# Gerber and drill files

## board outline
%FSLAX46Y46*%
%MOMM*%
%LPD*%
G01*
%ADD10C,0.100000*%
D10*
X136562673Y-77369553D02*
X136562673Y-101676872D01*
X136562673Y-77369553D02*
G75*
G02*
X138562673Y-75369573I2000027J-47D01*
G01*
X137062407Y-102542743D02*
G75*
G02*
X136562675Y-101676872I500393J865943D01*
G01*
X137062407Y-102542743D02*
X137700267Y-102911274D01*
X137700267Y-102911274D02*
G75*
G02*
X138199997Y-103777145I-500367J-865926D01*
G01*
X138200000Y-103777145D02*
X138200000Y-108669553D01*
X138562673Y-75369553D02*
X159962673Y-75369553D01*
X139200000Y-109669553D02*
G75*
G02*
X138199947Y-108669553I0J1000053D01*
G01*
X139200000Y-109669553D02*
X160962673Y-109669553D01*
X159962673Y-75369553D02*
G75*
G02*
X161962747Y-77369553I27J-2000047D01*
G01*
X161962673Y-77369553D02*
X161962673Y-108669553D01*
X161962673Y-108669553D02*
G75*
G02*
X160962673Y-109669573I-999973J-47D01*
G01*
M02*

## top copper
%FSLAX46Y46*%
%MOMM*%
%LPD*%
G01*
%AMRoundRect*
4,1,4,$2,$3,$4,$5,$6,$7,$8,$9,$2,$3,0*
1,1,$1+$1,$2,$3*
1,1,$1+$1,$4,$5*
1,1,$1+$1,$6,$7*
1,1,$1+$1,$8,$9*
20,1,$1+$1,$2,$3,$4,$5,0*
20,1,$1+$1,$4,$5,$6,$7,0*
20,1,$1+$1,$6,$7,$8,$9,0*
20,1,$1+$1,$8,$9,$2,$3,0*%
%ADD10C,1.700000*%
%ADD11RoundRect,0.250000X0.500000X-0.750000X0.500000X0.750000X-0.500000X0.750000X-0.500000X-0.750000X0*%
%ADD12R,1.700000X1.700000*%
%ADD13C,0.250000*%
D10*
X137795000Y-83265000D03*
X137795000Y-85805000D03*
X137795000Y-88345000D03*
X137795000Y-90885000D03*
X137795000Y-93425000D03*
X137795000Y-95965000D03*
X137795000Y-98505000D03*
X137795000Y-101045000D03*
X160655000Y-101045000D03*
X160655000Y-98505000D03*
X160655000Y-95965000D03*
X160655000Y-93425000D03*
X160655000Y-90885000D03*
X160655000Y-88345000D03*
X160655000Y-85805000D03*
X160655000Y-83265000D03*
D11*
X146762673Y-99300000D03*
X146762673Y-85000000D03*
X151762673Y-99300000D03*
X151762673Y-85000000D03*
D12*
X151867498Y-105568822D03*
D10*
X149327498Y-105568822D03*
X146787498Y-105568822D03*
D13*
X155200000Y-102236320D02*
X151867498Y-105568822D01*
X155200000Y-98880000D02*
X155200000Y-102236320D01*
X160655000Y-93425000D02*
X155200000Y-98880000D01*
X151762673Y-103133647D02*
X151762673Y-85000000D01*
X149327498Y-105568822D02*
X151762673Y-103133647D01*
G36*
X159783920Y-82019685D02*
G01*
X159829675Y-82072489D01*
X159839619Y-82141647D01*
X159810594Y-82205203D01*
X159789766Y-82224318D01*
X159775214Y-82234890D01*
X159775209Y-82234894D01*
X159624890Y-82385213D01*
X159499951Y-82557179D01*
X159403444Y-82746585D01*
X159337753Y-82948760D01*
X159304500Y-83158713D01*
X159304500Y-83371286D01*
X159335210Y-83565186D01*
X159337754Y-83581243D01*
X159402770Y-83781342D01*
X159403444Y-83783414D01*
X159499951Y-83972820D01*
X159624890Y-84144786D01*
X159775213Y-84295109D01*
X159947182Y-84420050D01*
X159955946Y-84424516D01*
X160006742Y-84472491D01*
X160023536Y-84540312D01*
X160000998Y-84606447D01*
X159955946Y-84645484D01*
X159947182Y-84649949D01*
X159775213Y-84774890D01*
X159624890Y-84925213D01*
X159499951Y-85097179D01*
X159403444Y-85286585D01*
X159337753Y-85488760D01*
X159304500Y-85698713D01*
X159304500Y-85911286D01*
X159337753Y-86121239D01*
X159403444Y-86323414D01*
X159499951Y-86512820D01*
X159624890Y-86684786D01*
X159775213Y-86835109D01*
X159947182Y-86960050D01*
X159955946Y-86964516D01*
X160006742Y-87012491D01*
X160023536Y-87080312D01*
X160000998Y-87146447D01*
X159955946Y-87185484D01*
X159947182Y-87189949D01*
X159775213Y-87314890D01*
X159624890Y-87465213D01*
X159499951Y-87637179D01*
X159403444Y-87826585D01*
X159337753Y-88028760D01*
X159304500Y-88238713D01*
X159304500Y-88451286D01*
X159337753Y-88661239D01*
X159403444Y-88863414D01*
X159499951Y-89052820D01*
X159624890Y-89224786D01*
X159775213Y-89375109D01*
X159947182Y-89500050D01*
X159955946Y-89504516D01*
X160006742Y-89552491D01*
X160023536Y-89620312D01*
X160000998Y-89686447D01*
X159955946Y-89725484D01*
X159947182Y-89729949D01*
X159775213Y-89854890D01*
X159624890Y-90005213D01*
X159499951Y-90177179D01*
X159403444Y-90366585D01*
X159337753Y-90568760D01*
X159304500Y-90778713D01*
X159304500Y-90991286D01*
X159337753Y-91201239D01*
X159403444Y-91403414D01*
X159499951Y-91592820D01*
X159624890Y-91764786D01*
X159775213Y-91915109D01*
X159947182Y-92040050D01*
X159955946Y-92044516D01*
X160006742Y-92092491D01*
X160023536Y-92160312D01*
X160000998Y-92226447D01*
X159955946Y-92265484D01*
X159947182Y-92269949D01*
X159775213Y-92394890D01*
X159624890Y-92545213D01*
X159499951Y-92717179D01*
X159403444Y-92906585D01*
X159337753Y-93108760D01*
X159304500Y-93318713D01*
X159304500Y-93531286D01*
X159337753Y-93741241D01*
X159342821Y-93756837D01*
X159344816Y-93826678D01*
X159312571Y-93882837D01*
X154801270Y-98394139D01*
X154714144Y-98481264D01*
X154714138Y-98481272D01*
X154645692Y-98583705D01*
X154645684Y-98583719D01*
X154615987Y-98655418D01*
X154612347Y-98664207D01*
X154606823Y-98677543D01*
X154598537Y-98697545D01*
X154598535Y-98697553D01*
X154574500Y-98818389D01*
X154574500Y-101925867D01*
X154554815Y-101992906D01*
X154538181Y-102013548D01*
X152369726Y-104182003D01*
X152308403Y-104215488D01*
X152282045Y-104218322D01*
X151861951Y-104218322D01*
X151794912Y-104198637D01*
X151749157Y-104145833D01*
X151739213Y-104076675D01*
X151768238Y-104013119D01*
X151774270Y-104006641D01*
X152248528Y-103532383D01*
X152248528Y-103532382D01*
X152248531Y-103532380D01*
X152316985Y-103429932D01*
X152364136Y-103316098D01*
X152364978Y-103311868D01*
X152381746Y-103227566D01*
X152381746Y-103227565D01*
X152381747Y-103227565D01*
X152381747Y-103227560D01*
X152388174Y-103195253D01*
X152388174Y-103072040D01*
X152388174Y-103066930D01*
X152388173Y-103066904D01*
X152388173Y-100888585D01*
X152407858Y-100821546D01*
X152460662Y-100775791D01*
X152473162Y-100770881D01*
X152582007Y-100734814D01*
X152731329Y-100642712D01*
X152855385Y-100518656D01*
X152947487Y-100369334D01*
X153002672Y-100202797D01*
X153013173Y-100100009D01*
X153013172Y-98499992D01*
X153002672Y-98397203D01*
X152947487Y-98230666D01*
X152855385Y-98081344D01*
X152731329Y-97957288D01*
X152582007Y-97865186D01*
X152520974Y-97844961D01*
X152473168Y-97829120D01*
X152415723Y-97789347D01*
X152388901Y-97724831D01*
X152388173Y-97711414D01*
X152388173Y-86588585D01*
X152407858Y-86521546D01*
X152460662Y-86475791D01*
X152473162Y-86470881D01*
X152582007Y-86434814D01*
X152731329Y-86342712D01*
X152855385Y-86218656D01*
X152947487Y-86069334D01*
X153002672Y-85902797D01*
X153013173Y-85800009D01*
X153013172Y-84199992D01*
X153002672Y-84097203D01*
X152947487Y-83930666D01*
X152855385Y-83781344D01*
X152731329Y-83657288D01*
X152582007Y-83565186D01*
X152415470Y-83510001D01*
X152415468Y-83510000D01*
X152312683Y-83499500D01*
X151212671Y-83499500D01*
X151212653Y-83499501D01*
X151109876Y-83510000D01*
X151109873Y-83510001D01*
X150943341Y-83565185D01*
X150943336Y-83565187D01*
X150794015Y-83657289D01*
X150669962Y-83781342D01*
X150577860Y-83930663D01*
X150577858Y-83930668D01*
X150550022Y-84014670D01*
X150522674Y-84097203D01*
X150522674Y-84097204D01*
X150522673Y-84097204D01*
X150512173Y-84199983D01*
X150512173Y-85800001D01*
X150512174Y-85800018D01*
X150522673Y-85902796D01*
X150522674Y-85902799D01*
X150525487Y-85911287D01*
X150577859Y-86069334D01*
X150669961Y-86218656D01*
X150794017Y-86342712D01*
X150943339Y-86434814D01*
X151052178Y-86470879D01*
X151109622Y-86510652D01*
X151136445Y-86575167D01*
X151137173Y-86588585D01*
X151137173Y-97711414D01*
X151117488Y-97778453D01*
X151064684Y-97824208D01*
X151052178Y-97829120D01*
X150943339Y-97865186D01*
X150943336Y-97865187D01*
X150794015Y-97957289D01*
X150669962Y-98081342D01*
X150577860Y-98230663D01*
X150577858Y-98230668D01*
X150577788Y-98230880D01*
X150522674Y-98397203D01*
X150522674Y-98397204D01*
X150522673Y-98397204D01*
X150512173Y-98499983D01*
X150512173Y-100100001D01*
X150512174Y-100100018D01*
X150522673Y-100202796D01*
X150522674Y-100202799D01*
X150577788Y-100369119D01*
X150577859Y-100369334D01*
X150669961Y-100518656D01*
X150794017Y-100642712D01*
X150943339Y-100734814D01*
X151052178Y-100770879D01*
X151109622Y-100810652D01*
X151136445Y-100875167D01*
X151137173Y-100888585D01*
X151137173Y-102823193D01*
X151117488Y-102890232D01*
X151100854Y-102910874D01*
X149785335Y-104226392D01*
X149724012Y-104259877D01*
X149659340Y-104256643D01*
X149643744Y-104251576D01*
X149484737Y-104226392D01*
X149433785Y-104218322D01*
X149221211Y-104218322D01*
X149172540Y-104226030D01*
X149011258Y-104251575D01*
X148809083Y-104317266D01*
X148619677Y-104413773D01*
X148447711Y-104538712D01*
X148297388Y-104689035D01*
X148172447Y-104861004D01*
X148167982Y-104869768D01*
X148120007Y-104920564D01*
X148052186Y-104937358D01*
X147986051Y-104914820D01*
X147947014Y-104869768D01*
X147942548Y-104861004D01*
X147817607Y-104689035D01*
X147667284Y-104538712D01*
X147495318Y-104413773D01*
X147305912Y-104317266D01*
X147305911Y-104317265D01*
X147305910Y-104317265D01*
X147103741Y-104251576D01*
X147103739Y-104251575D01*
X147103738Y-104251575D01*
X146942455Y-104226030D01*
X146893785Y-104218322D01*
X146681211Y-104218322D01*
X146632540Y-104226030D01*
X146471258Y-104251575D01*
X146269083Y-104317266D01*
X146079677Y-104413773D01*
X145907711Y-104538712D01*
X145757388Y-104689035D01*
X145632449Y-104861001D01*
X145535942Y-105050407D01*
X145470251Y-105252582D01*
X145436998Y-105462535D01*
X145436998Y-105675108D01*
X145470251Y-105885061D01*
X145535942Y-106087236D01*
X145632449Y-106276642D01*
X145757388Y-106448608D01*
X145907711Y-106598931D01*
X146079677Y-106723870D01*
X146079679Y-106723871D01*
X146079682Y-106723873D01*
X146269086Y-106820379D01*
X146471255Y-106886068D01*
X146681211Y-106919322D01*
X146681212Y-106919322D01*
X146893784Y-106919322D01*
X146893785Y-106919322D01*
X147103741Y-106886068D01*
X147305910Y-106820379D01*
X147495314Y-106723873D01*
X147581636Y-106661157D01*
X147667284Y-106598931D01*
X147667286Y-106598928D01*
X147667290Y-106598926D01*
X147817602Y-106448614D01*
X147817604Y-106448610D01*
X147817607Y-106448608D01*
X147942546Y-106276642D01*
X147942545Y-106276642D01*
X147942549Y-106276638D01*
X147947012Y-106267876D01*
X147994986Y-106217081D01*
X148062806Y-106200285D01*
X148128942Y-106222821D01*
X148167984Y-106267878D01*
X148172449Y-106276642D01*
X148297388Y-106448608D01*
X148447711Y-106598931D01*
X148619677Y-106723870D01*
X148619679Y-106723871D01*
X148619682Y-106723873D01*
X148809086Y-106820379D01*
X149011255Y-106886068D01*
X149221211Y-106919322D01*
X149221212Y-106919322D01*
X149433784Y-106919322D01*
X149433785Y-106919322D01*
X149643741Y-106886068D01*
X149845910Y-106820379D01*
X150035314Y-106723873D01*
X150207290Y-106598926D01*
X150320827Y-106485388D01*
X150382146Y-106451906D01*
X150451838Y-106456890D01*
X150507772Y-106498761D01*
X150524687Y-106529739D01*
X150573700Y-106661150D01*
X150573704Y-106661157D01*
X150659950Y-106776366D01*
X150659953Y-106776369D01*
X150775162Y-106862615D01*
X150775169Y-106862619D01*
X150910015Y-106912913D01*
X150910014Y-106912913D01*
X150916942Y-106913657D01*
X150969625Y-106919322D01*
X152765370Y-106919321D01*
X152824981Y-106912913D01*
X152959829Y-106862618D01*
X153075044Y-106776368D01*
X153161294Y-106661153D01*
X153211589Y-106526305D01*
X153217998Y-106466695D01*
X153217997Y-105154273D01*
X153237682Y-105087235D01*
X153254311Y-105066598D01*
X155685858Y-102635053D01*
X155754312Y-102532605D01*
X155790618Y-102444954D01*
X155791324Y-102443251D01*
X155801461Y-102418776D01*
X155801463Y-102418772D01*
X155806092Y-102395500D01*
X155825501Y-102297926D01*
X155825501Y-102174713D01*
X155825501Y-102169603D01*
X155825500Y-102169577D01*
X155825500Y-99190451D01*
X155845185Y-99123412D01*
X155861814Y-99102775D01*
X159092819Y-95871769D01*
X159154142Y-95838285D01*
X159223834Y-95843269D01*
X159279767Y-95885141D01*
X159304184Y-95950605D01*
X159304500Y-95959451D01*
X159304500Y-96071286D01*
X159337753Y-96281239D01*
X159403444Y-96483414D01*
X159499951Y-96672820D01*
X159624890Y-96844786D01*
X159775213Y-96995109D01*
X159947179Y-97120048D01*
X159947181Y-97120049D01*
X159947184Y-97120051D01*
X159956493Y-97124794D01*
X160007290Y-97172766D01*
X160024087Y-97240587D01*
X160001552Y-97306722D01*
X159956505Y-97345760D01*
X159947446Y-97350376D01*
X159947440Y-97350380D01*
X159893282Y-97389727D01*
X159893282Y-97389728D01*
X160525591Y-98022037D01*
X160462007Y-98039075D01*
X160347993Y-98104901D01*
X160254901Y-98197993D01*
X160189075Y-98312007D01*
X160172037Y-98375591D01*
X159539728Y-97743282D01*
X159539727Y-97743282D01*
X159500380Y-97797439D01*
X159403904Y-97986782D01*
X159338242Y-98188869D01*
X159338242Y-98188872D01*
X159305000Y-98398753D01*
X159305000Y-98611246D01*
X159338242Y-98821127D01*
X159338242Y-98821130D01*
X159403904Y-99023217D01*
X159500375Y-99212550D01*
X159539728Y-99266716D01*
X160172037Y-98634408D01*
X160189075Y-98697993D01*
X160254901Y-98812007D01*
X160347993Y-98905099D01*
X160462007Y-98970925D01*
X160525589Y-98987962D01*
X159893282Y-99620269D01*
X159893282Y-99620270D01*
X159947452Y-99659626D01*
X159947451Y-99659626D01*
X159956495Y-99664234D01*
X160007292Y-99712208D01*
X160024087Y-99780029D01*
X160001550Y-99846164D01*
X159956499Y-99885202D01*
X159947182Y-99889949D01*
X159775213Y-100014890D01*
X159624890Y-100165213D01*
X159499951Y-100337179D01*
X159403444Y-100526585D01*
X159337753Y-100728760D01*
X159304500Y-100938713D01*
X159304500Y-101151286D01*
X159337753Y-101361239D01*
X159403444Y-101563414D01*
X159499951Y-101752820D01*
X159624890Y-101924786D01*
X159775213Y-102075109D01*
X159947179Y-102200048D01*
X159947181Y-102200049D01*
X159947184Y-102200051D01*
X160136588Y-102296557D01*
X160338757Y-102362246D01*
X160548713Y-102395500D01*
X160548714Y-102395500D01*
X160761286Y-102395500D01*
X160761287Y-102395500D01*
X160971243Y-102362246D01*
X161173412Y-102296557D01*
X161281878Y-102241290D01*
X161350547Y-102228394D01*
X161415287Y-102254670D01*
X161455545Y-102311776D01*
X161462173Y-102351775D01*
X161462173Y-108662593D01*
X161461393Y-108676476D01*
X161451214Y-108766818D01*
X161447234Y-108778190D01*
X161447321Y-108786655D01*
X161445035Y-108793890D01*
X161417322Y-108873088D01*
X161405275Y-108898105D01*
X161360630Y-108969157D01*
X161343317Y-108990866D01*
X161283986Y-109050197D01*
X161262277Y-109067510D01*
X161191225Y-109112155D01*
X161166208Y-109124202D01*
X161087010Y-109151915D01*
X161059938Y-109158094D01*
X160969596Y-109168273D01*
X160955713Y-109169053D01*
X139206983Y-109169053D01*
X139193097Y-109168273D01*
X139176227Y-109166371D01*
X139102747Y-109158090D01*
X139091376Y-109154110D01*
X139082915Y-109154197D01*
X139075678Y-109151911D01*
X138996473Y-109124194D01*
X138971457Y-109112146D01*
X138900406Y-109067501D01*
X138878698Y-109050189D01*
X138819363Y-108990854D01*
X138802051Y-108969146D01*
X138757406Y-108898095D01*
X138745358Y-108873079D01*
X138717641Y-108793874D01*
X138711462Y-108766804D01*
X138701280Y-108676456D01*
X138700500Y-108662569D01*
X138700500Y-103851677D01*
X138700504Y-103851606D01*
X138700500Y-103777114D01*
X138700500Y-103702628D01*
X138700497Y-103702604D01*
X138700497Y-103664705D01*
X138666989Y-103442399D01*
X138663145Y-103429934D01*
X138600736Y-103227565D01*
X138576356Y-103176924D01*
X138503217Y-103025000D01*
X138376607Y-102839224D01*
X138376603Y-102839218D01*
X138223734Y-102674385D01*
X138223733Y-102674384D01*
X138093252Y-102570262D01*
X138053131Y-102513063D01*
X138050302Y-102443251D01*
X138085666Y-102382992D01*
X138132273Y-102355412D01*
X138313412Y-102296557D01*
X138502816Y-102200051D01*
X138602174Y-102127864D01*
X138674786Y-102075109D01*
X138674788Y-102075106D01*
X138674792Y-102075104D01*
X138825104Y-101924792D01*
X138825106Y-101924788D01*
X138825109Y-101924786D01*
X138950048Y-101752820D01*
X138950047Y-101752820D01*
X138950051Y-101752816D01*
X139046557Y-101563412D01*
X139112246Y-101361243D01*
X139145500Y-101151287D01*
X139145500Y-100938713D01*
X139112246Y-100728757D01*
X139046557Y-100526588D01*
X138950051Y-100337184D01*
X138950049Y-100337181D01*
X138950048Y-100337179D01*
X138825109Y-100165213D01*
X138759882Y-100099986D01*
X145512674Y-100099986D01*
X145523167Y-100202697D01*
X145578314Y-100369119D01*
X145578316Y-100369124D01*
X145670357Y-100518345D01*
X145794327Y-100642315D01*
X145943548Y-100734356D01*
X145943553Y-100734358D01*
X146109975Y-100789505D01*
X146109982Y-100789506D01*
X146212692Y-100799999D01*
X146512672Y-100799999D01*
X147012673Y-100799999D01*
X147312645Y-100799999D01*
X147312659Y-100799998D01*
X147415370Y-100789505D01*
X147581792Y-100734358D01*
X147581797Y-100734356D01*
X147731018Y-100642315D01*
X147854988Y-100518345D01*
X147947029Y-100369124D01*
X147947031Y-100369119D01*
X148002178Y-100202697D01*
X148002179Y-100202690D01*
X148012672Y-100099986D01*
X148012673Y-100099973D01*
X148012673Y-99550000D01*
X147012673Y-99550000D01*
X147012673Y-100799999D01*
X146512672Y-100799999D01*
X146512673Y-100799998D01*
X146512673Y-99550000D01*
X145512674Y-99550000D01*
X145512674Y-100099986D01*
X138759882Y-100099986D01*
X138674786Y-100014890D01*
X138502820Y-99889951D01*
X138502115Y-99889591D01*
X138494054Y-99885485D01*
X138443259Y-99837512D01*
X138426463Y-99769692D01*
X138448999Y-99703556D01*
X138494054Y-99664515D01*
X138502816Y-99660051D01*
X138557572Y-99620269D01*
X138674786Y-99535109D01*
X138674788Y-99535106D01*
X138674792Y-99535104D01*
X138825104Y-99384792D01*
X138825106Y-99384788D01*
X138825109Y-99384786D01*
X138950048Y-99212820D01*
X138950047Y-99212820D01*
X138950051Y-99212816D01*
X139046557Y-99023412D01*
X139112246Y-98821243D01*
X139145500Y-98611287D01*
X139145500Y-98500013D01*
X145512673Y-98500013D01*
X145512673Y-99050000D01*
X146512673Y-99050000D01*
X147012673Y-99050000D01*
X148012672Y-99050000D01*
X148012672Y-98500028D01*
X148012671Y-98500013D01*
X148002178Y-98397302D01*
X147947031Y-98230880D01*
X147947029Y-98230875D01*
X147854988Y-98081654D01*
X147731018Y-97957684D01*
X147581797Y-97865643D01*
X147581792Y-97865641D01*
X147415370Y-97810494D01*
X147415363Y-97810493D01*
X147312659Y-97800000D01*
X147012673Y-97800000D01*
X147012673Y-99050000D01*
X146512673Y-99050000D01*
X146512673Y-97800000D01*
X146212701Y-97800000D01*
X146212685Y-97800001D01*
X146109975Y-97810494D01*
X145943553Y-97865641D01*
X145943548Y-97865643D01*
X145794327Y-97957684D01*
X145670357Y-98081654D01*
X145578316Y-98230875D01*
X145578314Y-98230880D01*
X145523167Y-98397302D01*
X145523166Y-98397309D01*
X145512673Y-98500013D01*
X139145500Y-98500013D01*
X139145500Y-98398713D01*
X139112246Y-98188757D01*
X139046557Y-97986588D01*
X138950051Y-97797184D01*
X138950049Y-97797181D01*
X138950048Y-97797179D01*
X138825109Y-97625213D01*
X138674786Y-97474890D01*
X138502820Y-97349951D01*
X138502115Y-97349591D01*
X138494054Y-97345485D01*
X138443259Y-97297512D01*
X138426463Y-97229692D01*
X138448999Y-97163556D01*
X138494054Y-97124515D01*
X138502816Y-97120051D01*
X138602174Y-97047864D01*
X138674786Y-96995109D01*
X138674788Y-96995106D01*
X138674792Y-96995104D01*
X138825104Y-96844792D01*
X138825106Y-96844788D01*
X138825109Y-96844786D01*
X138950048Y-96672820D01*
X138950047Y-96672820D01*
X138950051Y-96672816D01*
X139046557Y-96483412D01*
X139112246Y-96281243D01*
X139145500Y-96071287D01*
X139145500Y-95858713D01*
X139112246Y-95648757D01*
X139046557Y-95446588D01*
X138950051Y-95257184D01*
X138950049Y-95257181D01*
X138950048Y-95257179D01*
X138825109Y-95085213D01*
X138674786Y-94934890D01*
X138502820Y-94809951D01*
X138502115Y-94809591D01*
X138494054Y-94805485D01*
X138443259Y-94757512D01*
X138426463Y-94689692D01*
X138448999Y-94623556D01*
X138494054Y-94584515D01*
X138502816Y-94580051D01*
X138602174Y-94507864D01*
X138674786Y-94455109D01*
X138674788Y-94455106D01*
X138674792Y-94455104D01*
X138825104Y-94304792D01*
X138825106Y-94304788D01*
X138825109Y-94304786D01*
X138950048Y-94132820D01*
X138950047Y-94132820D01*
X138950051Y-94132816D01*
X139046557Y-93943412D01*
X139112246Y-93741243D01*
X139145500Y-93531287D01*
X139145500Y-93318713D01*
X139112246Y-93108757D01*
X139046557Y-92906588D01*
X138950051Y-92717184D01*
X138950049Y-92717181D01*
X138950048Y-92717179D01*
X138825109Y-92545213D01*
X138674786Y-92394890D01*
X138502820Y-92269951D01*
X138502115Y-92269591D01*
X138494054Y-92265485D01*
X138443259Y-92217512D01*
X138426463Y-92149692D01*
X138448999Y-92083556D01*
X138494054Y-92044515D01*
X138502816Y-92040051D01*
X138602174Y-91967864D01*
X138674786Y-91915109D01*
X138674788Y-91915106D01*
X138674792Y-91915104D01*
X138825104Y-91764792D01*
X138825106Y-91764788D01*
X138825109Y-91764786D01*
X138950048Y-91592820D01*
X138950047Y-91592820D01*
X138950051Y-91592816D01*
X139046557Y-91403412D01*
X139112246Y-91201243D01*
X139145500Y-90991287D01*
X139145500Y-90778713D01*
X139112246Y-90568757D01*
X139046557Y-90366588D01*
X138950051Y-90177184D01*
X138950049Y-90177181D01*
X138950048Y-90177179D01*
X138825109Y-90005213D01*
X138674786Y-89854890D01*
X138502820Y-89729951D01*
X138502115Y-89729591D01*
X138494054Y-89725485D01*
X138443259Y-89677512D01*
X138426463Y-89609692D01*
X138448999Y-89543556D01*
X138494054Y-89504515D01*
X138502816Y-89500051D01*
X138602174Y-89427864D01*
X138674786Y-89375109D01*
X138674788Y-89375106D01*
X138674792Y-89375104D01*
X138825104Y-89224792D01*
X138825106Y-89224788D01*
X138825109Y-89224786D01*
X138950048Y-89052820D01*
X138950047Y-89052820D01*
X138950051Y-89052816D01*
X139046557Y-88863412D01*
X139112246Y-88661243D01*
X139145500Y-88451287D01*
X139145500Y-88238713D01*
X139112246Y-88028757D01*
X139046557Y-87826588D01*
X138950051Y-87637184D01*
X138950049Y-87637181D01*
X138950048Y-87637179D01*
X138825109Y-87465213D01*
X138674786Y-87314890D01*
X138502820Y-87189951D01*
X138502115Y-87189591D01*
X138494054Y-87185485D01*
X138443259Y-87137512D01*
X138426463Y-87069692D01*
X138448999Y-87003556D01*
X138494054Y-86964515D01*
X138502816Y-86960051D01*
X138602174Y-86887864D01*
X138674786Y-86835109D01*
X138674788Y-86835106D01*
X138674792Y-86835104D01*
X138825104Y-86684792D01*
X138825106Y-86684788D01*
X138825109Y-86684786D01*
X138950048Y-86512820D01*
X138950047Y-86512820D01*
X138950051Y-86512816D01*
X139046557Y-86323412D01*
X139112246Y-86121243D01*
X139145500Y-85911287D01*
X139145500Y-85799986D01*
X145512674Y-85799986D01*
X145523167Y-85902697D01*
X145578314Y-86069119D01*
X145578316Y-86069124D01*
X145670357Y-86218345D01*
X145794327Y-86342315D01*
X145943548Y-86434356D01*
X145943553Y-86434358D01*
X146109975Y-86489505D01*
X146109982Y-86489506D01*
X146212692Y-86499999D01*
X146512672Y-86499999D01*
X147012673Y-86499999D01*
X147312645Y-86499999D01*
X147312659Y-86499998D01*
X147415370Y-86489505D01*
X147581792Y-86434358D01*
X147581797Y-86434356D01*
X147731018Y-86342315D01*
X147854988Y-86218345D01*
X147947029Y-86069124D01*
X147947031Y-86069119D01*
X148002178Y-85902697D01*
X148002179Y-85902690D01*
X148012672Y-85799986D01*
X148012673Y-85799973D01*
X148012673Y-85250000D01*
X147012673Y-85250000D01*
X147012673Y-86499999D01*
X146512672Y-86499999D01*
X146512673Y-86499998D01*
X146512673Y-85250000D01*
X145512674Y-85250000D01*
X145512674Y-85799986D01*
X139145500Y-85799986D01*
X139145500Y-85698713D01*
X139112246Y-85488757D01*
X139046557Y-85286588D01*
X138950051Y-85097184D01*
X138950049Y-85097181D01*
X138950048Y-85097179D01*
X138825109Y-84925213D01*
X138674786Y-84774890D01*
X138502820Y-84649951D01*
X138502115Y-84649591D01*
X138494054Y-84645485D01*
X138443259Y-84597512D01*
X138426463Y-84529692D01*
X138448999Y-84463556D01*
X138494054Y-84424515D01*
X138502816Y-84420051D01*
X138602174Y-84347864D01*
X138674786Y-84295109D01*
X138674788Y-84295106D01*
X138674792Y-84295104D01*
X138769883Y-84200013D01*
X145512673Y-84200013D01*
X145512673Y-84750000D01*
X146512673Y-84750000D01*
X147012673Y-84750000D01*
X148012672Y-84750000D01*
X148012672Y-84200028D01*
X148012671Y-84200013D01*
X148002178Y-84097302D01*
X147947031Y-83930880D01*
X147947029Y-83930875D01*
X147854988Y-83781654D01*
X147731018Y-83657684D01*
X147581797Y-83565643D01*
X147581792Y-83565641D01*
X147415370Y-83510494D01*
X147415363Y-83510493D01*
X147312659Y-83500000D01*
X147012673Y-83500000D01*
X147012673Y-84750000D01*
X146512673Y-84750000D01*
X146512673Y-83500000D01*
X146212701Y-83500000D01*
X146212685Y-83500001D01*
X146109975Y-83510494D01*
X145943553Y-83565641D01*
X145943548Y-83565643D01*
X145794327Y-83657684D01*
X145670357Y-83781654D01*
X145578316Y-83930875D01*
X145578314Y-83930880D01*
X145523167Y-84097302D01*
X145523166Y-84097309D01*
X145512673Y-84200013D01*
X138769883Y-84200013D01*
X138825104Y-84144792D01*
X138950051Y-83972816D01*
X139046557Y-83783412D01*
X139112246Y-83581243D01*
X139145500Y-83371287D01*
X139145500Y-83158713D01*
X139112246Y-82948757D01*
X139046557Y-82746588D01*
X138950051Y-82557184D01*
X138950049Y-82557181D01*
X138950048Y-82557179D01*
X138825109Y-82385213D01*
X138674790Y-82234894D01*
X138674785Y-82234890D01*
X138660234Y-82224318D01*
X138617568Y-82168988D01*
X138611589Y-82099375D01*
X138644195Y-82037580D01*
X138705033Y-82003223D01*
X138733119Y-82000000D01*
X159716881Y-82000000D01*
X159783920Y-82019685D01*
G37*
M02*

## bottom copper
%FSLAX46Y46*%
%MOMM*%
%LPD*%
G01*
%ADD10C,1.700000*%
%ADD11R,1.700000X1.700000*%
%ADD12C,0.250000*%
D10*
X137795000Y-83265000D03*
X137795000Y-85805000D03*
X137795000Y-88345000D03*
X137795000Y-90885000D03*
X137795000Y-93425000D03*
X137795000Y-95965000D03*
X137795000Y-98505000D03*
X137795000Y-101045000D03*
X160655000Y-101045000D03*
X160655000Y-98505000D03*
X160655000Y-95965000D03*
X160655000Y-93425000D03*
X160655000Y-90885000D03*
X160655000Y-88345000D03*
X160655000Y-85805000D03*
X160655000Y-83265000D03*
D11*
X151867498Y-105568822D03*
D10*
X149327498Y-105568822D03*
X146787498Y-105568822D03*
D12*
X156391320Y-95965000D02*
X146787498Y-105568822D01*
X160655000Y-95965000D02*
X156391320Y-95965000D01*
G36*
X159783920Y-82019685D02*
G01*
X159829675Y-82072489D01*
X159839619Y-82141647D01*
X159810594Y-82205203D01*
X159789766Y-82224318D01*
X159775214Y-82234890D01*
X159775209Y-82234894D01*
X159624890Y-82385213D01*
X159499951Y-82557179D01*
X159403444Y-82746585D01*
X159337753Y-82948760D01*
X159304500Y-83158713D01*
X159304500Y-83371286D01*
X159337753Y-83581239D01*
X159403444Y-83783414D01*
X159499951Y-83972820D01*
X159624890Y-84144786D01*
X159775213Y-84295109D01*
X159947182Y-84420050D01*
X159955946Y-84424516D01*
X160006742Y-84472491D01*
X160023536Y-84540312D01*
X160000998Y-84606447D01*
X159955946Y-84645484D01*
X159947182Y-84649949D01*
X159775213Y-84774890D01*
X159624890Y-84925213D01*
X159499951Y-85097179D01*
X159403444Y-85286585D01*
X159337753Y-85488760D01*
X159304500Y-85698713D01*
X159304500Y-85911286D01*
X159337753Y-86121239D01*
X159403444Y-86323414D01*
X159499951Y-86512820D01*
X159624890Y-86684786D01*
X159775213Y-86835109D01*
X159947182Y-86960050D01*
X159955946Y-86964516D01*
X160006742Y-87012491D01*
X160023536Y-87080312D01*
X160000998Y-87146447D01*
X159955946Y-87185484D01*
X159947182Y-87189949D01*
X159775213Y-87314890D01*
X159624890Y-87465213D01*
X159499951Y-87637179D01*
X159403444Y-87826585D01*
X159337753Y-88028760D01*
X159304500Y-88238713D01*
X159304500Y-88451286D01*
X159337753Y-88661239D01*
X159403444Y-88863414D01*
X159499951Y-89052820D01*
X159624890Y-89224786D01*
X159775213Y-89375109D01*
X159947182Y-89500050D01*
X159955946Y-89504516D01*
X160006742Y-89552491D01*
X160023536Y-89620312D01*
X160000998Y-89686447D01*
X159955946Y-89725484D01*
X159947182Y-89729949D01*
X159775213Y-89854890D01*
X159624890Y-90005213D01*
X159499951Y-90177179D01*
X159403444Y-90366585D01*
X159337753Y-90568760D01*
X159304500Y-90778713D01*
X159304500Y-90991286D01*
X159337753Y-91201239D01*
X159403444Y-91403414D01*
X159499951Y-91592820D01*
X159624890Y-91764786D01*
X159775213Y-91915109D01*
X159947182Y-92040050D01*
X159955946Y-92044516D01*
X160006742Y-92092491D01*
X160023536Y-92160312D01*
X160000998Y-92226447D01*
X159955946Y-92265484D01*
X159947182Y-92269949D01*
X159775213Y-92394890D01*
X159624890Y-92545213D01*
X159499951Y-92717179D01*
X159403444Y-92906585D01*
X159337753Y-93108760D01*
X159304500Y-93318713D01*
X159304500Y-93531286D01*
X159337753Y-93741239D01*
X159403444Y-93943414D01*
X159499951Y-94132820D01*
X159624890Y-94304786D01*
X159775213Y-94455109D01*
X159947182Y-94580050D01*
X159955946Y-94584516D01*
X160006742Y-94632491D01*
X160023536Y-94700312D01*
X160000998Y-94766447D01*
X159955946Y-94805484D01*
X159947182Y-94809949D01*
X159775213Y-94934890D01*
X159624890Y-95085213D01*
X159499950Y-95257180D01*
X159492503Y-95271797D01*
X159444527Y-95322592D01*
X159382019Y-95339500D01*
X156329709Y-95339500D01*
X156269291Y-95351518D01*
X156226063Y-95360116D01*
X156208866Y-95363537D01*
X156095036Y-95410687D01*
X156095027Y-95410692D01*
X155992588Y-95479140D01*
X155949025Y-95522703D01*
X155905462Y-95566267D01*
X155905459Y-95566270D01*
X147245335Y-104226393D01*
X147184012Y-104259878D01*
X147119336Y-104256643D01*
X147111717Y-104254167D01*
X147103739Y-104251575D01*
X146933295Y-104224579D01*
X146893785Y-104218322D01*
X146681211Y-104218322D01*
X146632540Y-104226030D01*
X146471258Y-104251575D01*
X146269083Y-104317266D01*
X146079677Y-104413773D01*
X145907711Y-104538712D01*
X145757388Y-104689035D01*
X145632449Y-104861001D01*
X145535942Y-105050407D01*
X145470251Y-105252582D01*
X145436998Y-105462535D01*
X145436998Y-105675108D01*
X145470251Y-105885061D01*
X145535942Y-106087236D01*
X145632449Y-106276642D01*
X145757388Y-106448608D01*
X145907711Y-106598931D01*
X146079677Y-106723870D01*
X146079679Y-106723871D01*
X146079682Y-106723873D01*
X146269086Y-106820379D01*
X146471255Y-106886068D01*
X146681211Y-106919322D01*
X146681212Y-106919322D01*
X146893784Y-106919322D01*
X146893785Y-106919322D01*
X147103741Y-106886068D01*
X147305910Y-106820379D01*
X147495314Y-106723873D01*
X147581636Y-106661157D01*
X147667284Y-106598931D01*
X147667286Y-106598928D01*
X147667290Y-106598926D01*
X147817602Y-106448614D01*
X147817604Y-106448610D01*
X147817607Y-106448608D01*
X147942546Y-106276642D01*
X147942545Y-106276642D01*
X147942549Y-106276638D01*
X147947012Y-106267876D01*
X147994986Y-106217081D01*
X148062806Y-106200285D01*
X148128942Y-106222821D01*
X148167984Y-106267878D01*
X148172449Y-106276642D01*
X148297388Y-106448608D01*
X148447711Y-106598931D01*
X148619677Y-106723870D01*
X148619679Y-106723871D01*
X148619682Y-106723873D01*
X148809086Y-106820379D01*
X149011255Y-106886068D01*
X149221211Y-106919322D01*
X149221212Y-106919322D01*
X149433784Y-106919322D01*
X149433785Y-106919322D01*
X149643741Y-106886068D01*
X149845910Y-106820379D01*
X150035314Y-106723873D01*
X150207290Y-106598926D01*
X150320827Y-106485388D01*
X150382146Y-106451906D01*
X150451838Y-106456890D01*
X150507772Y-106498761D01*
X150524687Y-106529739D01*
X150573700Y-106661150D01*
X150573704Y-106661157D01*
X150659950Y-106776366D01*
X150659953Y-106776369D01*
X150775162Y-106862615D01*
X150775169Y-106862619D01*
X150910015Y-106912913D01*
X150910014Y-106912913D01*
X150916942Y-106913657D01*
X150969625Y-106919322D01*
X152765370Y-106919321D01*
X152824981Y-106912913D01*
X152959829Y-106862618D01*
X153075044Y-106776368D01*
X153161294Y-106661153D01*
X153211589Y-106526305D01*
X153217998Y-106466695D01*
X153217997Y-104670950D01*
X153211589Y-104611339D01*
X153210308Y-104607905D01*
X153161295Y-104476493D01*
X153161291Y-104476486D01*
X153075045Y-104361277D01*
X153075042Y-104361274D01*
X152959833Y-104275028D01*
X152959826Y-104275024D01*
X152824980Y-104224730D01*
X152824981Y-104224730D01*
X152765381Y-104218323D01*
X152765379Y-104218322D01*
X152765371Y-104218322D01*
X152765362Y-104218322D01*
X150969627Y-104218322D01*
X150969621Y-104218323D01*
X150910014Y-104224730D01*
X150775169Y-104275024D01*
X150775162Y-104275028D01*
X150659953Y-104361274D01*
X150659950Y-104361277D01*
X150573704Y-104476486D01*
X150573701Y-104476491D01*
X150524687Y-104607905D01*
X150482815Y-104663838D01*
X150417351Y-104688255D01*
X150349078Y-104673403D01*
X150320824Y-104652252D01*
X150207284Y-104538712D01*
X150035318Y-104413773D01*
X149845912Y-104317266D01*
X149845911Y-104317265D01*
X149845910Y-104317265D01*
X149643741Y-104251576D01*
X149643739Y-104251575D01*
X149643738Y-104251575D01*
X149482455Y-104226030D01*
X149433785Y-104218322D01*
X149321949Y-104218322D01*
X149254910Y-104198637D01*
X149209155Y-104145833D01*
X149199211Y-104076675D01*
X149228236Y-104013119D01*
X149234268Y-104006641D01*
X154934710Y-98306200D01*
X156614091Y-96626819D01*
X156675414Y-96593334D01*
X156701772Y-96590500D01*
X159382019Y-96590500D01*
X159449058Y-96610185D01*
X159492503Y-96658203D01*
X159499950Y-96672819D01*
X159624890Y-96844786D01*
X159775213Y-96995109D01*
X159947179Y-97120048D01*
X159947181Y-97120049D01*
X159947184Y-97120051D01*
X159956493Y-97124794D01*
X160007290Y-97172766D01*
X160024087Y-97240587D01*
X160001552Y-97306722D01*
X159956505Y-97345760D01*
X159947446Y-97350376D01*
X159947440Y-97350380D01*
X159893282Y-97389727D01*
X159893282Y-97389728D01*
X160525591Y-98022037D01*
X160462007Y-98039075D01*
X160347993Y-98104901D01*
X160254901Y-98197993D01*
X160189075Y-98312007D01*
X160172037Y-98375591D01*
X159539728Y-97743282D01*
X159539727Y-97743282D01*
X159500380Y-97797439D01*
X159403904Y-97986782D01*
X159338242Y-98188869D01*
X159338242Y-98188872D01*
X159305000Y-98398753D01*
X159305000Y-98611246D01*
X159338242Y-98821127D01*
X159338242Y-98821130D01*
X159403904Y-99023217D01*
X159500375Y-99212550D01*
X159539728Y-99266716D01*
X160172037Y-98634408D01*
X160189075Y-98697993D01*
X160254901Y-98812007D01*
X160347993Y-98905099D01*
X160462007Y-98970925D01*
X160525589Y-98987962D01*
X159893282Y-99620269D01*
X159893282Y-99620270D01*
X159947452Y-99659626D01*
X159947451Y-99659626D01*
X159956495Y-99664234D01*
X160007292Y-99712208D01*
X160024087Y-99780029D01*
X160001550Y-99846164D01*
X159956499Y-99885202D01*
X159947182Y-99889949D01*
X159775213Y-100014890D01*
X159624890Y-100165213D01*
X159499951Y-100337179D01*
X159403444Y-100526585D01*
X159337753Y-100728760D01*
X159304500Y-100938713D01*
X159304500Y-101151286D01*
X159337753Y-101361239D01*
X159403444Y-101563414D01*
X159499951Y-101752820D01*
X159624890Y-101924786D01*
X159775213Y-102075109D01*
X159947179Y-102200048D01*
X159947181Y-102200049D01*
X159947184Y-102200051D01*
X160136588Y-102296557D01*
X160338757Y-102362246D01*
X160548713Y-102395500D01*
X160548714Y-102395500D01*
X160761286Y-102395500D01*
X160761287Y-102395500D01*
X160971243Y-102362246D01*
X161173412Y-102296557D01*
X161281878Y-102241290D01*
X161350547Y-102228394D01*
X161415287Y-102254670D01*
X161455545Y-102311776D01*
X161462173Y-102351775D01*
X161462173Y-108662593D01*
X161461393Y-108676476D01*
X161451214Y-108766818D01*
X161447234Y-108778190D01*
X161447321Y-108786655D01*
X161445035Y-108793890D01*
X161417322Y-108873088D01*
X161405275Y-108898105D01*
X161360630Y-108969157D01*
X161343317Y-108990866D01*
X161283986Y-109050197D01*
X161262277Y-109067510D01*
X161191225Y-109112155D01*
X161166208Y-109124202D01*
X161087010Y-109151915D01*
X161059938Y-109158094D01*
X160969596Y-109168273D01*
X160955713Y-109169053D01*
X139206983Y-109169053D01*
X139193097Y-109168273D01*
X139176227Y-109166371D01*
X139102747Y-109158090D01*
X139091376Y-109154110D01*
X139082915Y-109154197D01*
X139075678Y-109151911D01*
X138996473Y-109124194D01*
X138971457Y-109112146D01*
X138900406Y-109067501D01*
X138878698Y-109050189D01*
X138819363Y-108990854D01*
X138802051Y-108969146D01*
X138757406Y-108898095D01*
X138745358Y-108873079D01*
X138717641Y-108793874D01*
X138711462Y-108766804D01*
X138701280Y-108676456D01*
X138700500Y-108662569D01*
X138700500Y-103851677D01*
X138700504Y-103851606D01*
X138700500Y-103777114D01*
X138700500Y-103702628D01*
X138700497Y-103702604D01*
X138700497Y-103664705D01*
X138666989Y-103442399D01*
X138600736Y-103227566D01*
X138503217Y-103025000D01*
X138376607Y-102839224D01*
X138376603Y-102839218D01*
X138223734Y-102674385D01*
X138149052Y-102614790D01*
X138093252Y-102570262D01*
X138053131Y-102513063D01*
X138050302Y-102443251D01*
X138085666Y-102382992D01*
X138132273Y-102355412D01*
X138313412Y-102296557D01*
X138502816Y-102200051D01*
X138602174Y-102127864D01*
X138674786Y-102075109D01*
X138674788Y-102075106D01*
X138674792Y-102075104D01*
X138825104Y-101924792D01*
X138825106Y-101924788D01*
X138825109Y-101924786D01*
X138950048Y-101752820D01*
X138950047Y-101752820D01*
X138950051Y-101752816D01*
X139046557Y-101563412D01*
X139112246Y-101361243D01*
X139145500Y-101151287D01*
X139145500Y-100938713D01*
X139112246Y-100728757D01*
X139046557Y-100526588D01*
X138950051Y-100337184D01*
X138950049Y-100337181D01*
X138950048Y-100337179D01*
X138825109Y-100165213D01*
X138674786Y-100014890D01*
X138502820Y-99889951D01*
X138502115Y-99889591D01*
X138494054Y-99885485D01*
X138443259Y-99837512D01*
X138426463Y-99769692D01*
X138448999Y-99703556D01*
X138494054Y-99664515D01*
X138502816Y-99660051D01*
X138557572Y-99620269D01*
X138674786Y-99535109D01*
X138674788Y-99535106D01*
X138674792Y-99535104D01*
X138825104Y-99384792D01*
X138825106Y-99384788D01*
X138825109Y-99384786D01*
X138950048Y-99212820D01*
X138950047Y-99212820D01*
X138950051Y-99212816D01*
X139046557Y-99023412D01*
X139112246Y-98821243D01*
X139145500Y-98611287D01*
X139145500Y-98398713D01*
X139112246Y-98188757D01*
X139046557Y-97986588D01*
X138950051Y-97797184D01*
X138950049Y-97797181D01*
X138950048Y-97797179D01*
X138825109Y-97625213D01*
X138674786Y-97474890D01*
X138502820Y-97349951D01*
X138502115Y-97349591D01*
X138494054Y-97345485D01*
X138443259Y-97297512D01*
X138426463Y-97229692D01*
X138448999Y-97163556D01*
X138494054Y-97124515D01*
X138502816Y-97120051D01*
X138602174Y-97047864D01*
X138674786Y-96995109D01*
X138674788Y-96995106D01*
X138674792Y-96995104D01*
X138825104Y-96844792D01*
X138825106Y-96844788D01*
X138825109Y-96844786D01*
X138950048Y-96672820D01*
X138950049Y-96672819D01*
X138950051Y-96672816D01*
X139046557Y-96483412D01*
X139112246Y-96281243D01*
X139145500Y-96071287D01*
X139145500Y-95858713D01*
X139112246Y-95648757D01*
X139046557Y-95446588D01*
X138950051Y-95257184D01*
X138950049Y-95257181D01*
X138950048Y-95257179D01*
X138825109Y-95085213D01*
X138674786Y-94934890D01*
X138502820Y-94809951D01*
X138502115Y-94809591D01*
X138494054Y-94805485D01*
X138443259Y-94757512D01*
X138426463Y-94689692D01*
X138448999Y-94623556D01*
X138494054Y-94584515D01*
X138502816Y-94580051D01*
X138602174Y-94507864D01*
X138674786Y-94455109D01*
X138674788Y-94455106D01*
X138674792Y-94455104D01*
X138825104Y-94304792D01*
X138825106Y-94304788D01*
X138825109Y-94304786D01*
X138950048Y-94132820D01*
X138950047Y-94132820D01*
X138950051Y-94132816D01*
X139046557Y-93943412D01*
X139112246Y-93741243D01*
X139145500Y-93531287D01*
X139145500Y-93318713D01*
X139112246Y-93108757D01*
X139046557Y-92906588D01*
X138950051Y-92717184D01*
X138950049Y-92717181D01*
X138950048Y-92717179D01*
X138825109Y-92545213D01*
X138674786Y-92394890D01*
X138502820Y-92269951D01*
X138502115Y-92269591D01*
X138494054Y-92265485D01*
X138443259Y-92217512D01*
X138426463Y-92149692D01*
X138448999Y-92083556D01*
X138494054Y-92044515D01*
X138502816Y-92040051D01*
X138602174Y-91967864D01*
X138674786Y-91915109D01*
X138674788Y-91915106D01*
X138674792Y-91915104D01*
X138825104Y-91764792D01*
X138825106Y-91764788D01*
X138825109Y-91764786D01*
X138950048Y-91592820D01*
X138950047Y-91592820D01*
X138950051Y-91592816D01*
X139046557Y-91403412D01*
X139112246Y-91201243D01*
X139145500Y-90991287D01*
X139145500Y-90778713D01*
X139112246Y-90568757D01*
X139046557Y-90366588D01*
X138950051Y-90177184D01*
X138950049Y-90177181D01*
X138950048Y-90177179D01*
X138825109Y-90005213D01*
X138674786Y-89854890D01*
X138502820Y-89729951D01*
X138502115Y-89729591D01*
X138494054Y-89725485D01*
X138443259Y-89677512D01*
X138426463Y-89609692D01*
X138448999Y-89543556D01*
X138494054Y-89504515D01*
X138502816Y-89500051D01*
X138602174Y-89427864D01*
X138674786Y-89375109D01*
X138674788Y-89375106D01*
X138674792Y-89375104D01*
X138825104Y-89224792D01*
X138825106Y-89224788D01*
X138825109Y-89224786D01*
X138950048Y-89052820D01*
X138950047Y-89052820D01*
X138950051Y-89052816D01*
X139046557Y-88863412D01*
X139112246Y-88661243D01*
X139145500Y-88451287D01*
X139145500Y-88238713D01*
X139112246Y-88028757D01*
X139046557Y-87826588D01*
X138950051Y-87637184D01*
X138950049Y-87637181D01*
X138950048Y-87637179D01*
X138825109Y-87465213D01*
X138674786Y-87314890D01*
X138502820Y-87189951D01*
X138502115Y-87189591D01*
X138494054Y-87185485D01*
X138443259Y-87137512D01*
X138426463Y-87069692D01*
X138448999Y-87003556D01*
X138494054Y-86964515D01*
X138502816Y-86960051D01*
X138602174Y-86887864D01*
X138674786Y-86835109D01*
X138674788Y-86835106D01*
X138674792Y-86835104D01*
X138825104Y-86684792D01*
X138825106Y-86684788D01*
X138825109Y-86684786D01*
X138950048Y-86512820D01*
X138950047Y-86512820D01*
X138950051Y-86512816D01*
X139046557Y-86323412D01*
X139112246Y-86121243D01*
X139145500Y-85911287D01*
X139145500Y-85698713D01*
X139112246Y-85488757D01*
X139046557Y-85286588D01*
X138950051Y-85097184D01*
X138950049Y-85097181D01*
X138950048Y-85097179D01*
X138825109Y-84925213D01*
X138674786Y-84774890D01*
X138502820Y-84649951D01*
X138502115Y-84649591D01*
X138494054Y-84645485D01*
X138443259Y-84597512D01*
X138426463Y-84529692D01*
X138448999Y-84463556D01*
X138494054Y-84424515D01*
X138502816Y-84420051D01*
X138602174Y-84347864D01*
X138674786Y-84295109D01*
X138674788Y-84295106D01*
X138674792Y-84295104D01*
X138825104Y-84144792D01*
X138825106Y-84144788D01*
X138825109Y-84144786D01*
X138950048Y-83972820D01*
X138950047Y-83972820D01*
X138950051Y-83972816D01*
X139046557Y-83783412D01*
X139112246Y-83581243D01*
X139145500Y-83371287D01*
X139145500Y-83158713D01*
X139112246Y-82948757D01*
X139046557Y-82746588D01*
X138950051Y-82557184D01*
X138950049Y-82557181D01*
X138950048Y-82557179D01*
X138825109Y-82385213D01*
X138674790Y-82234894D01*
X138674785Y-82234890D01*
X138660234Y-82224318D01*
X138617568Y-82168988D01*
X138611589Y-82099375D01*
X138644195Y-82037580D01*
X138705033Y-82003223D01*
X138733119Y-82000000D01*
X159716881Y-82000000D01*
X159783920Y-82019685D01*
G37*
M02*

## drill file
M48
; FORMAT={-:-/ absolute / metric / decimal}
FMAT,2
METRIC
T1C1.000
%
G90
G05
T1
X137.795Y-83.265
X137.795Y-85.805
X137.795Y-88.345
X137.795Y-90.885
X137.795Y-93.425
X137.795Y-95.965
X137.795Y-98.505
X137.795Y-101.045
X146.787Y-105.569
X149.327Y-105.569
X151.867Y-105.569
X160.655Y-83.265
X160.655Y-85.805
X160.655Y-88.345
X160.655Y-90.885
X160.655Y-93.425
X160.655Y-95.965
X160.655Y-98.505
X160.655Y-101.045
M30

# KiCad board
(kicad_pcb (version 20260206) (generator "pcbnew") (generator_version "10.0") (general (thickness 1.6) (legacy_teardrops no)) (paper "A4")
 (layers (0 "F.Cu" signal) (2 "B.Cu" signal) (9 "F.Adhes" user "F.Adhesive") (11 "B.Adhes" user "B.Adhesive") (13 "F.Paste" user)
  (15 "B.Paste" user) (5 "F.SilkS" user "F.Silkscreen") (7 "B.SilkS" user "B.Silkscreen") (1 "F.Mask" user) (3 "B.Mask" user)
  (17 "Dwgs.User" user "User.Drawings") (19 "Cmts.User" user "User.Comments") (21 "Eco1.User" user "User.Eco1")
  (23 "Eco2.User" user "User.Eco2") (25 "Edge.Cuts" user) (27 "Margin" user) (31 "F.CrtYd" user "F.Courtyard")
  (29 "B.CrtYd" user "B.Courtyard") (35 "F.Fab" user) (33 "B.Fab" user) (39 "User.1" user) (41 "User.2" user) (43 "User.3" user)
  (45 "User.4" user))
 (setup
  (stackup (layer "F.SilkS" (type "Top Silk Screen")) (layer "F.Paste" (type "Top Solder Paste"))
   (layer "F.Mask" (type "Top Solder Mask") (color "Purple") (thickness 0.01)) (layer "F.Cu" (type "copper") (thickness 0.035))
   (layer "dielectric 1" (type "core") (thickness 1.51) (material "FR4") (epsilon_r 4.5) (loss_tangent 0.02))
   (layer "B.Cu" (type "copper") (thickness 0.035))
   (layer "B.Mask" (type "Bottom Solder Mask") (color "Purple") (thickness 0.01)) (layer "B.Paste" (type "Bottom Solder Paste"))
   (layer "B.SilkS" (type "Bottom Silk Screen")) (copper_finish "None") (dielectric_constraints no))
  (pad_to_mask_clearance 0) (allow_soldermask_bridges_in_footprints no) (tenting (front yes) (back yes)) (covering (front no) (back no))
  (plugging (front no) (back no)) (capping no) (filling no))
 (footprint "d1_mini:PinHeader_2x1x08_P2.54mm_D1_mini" (layer "F.Cu") (at 137.795 83.045)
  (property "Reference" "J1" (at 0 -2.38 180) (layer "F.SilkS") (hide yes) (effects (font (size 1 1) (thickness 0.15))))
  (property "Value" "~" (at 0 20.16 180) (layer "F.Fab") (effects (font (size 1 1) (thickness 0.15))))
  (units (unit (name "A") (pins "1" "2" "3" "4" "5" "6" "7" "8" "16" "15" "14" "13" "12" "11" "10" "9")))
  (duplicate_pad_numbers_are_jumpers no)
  (pad "1" thru_hole circle (at 0 0.22 180) (size 1.7 1.7) (drill 1) (layers "*.Cu" "*.Mask") (remove_unused_layers no)
   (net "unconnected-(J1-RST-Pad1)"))
  (pad "2" thru_hole circle (at 0 2.76 180) (size 1.7 1.7) (drill 1) (layers "*.Cu" "*.Mask") (remove_unused_layers no)
   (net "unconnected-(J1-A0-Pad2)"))
  (pad "3" thru_hole circle (at 0 5.3 180) (size 1.7 1.7) (drill 1) (layers "*.Cu" "*.Mask") (remove_unused_layers no)
   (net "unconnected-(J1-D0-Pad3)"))
  (pad "4" thru_hole circle (at 0 7.84 180) (size 1.7 1.7) (drill 1) (layers "*.Cu" "*.Mask") (remove_unused_layers no)
   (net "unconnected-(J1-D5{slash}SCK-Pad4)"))
  (pad "5" thru_hole circle (at 0 10.38 180) (size 1.7 1.7) (drill 1) (layers "*.Cu" "*.Mask") (remove_unused_layers no)
   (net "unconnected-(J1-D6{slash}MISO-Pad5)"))
  (pad "6" thru_hole circle (at 0 12.92 180) (size 1.7 1.7) (drill 1) (layers "*.Cu" "*.Mask") (remove_unused_layers no)
   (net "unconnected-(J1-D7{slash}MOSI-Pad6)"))
  (pad "7" thru_hole circle (at 0 15.46 180) (size 1.7 1.7) (drill 1) (layers "*.Cu" "*.Mask") (remove_unused_layers no)
   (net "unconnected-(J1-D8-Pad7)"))
  (pad "8" thru_hole circle (at 0 18 180) (size 1.7 1.7) (drill 1) (layers "*.Cu" "*.Mask") (remove_unused_layers no)
   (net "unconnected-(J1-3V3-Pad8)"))
  (pad "9" thru_hole circle (at 22.86 18 180) (size 1.7 1.7) (drill 1) (layers "*.Cu" "*.Mask") (remove_unused_layers no)
   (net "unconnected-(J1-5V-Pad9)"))
  (pad "10" thru_hole circle (at 22.86 15.46 180) (size 1.7 1.7) (drill 1) (layers "*.Cu" "*.Mask") (remove_unused_layers no) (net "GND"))
  (pad "11" thru_hole circle (at 22.86 12.92 180) (size 1.7 1.7) (drill 1) (layers "*.Cu" "*.Mask") (remove_unused_layers no) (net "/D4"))
  (pad "12" thru_hole circle (at 22.86 10.38 180) (size 1.7 1.7) (drill 1) (layers "*.Cu" "*.Mask") (remove_unused_layers no) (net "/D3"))
  (pad "13" thru_hole circle (at 22.86 7.84 180) (size 1.7 1.7) (drill 1) (layers "*.Cu" "*.Mask") (remove_unused_layers no)
   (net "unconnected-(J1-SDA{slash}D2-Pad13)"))
  (pad "14" thru_hole circle (at 22.86 5.3 180) (size 1.7 1.7) (drill 1) (layers "*.Cu" "*.Mask") (remove_unused_layers no)
   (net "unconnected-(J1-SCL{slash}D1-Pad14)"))
  (pad "15" thru_hole circle (at 22.86 2.76 180) (size 1.7 1.7) (drill 1) (layers "*.Cu" "*.Mask") (remove_unused_layers no)
   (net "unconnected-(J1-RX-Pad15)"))
  (pad "16" thru_hole circle (at 22.86 0.22 180) (size 1.7 1.7) (drill 1) (layers "*.Cu" "*.Mask") (remove_unused_layers no)
   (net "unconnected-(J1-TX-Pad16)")))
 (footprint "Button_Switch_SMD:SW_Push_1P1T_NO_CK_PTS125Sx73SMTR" (layer "F.Cu") (at 149.262673 92.15 90)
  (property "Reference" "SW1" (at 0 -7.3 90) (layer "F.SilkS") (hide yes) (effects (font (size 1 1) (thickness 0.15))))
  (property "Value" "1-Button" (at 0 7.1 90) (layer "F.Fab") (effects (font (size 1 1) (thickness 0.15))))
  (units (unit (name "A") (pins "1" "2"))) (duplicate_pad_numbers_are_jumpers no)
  (pad "1" smd roundrect (at -7.15 -2.5 90) (size 2 1.5) (layers "F.Cu" "F.Mask" "F.Paste") (roundrect_rratio 0.1666666667) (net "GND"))
  (pad "1" smd roundrect (at 7.15 -2.5 90) (size 2 1.5) (layers "F.Cu" "F.Mask" "F.Paste") (roundrect_rratio 0.1666666667) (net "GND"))
  (pad "2" smd roundrect (at -7.15 2.5 90) (size 2 1.5) (layers "F.Cu" "F.Mask" "F.Paste") (roundrect_rratio 0.1666666667)
   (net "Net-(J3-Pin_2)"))
  (pad "2" smd roundrect (at 7.15 2.5 90) (size 2 1.5) (layers "F.Cu" "F.Mask" "F.Paste") (roundrect_rratio 0.1666666667)
   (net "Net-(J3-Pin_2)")))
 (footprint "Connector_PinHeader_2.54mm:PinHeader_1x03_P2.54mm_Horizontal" (layer "B.Cu") (at 151.867498 105.568822 90)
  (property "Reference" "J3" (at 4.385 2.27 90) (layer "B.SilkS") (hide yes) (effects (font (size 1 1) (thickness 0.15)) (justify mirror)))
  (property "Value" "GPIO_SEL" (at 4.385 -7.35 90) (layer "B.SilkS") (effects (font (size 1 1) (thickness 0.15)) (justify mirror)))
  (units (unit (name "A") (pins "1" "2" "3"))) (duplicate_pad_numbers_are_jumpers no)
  (pad "1" thru_hole rect (at 0 0 90) (size 1.7 1.7) (drill 1) (layers "*.Cu" "*.Mask") (remove_unused_layers no) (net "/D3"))
  (pad "2" thru_hole circle (at 0 -2.54 90) (size 1.7 1.7) (drill 1) (layers "*.Cu" "*.Mask") (remove_unused_layers no)
   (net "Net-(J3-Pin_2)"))
  (pad "3" thru_hole circle (at 0 -5.08 90) (size 1.7 1.7) (drill 1) (layers "*.Cu" "*.Mask") (remove_unused_layers no) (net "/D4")))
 (gr_line (start 136.562673 77.369553) (end 136.562673 101.676872) (stroke (width 0.1) (type solid)) (layer "Edge.Cuts"))
 (gr_arc (start 136.562673 77.369553) (mid 137.148459 75.955339) (end 138.562673 75.369553) (stroke (width 0.1) (type default))
  (layer "Edge.Cuts"))
 (gr_arc (start 137.062407 102.542743) (mid 136.696591 102.176733) (end 136.562673 101.676872) (stroke (width 0.1) (type default))
  (layer "Edge.Cuts"))
 (gr_line (start 137.062407 102.542743) (end 137.700267 102.911274) (stroke (width 0.1) (type solid)) (layer "Edge.Cuts"))
 (gr_arc (start 137.700267 102.911274) (mid 138.066085 103.277282) (end 138.2 103.777145) (stroke (width 0.1) (type default))
  (layer "Edge.Cuts"))
 (gr_line (start 138.2 103.777145) (end 138.2 108.669553) (stroke (width 0.1) (type solid)) (layer "Edge.Cuts"))
 (gr_line (start 138.562673 75.369553) (end 159.962673 75.369553) (stroke (width 0.1) (type solid)) (layer "Edge.Cuts"))
 (gr_arc (start 139.2 109.669553) (mid 138.49291 109.376657) (end 138.2 108.669553) (stroke (width 0.1) (type default)) (layer "Edge.Cuts"))
 (gr_line (start 139.2 109.669553) (end 160.962673 109.669553) (stroke (width 0.1) (type solid)) (layer "Edge.Cuts"))
 (gr_arc (start 159.962673 75.369553) (mid 161.376887 75.955339) (end 161.962673 77.369553) (stroke (width 0.1) (type default))
  (layer "Edge.Cuts"))
 (gr_line (start 161.962673 77.369553) (end 161.962673 108.669553) (stroke (width 0.1) (type solid)) (layer "Edge.Cuts"))
 (gr_arc (start 161.962673 108.669553) (mid 161.66978 109.37666) (end 160.962673 109.669553) (stroke (width 0.1) (type default))
  (layer "Edge.Cuts"))
 (segment (start 156.39132 95.965) (end 146.787498 105.568822) (width 0.25) (layer "B.Cu") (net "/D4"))
 (segment (start 160.655 95.965) (end 156.39132 95.965) (width 0.25) (layer "B.Cu") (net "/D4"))
 (segment (start 155.2 102.23632) (end 151.867498 105.568822) (width 0.25) (layer "F.Cu") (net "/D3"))
 (segment (start 155.2 98.88) (end 155.2 102.23632) (width 0.25) (layer "F.Cu") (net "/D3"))
 (segment (start 160.655 93.425) (end 155.2 98.88) (width 0.25) (layer "F.Cu") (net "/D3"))
 (segment (start 151.762673 103.133647) (end 151.762673 85) (width 0.25) (layer "F.Cu") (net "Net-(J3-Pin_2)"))
 (segment (start 149.327498 105.568822) (end 151.762673 103.133647) (width 0.25) (layer "F.Cu") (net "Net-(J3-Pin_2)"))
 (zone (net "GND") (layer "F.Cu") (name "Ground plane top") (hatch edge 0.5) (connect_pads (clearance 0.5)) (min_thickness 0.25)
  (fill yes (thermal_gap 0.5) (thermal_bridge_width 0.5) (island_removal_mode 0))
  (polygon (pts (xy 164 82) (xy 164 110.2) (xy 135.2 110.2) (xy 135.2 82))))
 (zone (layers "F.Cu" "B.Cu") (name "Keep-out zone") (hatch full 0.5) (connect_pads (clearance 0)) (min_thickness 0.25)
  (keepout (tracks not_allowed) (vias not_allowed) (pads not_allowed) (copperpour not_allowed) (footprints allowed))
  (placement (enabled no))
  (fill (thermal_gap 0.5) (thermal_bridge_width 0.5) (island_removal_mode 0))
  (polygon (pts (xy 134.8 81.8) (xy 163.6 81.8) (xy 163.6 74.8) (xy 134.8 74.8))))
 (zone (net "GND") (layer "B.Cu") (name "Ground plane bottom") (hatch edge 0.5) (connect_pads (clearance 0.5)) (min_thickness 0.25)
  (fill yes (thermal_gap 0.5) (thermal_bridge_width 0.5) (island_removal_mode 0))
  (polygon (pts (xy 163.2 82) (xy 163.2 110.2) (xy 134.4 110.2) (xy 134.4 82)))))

